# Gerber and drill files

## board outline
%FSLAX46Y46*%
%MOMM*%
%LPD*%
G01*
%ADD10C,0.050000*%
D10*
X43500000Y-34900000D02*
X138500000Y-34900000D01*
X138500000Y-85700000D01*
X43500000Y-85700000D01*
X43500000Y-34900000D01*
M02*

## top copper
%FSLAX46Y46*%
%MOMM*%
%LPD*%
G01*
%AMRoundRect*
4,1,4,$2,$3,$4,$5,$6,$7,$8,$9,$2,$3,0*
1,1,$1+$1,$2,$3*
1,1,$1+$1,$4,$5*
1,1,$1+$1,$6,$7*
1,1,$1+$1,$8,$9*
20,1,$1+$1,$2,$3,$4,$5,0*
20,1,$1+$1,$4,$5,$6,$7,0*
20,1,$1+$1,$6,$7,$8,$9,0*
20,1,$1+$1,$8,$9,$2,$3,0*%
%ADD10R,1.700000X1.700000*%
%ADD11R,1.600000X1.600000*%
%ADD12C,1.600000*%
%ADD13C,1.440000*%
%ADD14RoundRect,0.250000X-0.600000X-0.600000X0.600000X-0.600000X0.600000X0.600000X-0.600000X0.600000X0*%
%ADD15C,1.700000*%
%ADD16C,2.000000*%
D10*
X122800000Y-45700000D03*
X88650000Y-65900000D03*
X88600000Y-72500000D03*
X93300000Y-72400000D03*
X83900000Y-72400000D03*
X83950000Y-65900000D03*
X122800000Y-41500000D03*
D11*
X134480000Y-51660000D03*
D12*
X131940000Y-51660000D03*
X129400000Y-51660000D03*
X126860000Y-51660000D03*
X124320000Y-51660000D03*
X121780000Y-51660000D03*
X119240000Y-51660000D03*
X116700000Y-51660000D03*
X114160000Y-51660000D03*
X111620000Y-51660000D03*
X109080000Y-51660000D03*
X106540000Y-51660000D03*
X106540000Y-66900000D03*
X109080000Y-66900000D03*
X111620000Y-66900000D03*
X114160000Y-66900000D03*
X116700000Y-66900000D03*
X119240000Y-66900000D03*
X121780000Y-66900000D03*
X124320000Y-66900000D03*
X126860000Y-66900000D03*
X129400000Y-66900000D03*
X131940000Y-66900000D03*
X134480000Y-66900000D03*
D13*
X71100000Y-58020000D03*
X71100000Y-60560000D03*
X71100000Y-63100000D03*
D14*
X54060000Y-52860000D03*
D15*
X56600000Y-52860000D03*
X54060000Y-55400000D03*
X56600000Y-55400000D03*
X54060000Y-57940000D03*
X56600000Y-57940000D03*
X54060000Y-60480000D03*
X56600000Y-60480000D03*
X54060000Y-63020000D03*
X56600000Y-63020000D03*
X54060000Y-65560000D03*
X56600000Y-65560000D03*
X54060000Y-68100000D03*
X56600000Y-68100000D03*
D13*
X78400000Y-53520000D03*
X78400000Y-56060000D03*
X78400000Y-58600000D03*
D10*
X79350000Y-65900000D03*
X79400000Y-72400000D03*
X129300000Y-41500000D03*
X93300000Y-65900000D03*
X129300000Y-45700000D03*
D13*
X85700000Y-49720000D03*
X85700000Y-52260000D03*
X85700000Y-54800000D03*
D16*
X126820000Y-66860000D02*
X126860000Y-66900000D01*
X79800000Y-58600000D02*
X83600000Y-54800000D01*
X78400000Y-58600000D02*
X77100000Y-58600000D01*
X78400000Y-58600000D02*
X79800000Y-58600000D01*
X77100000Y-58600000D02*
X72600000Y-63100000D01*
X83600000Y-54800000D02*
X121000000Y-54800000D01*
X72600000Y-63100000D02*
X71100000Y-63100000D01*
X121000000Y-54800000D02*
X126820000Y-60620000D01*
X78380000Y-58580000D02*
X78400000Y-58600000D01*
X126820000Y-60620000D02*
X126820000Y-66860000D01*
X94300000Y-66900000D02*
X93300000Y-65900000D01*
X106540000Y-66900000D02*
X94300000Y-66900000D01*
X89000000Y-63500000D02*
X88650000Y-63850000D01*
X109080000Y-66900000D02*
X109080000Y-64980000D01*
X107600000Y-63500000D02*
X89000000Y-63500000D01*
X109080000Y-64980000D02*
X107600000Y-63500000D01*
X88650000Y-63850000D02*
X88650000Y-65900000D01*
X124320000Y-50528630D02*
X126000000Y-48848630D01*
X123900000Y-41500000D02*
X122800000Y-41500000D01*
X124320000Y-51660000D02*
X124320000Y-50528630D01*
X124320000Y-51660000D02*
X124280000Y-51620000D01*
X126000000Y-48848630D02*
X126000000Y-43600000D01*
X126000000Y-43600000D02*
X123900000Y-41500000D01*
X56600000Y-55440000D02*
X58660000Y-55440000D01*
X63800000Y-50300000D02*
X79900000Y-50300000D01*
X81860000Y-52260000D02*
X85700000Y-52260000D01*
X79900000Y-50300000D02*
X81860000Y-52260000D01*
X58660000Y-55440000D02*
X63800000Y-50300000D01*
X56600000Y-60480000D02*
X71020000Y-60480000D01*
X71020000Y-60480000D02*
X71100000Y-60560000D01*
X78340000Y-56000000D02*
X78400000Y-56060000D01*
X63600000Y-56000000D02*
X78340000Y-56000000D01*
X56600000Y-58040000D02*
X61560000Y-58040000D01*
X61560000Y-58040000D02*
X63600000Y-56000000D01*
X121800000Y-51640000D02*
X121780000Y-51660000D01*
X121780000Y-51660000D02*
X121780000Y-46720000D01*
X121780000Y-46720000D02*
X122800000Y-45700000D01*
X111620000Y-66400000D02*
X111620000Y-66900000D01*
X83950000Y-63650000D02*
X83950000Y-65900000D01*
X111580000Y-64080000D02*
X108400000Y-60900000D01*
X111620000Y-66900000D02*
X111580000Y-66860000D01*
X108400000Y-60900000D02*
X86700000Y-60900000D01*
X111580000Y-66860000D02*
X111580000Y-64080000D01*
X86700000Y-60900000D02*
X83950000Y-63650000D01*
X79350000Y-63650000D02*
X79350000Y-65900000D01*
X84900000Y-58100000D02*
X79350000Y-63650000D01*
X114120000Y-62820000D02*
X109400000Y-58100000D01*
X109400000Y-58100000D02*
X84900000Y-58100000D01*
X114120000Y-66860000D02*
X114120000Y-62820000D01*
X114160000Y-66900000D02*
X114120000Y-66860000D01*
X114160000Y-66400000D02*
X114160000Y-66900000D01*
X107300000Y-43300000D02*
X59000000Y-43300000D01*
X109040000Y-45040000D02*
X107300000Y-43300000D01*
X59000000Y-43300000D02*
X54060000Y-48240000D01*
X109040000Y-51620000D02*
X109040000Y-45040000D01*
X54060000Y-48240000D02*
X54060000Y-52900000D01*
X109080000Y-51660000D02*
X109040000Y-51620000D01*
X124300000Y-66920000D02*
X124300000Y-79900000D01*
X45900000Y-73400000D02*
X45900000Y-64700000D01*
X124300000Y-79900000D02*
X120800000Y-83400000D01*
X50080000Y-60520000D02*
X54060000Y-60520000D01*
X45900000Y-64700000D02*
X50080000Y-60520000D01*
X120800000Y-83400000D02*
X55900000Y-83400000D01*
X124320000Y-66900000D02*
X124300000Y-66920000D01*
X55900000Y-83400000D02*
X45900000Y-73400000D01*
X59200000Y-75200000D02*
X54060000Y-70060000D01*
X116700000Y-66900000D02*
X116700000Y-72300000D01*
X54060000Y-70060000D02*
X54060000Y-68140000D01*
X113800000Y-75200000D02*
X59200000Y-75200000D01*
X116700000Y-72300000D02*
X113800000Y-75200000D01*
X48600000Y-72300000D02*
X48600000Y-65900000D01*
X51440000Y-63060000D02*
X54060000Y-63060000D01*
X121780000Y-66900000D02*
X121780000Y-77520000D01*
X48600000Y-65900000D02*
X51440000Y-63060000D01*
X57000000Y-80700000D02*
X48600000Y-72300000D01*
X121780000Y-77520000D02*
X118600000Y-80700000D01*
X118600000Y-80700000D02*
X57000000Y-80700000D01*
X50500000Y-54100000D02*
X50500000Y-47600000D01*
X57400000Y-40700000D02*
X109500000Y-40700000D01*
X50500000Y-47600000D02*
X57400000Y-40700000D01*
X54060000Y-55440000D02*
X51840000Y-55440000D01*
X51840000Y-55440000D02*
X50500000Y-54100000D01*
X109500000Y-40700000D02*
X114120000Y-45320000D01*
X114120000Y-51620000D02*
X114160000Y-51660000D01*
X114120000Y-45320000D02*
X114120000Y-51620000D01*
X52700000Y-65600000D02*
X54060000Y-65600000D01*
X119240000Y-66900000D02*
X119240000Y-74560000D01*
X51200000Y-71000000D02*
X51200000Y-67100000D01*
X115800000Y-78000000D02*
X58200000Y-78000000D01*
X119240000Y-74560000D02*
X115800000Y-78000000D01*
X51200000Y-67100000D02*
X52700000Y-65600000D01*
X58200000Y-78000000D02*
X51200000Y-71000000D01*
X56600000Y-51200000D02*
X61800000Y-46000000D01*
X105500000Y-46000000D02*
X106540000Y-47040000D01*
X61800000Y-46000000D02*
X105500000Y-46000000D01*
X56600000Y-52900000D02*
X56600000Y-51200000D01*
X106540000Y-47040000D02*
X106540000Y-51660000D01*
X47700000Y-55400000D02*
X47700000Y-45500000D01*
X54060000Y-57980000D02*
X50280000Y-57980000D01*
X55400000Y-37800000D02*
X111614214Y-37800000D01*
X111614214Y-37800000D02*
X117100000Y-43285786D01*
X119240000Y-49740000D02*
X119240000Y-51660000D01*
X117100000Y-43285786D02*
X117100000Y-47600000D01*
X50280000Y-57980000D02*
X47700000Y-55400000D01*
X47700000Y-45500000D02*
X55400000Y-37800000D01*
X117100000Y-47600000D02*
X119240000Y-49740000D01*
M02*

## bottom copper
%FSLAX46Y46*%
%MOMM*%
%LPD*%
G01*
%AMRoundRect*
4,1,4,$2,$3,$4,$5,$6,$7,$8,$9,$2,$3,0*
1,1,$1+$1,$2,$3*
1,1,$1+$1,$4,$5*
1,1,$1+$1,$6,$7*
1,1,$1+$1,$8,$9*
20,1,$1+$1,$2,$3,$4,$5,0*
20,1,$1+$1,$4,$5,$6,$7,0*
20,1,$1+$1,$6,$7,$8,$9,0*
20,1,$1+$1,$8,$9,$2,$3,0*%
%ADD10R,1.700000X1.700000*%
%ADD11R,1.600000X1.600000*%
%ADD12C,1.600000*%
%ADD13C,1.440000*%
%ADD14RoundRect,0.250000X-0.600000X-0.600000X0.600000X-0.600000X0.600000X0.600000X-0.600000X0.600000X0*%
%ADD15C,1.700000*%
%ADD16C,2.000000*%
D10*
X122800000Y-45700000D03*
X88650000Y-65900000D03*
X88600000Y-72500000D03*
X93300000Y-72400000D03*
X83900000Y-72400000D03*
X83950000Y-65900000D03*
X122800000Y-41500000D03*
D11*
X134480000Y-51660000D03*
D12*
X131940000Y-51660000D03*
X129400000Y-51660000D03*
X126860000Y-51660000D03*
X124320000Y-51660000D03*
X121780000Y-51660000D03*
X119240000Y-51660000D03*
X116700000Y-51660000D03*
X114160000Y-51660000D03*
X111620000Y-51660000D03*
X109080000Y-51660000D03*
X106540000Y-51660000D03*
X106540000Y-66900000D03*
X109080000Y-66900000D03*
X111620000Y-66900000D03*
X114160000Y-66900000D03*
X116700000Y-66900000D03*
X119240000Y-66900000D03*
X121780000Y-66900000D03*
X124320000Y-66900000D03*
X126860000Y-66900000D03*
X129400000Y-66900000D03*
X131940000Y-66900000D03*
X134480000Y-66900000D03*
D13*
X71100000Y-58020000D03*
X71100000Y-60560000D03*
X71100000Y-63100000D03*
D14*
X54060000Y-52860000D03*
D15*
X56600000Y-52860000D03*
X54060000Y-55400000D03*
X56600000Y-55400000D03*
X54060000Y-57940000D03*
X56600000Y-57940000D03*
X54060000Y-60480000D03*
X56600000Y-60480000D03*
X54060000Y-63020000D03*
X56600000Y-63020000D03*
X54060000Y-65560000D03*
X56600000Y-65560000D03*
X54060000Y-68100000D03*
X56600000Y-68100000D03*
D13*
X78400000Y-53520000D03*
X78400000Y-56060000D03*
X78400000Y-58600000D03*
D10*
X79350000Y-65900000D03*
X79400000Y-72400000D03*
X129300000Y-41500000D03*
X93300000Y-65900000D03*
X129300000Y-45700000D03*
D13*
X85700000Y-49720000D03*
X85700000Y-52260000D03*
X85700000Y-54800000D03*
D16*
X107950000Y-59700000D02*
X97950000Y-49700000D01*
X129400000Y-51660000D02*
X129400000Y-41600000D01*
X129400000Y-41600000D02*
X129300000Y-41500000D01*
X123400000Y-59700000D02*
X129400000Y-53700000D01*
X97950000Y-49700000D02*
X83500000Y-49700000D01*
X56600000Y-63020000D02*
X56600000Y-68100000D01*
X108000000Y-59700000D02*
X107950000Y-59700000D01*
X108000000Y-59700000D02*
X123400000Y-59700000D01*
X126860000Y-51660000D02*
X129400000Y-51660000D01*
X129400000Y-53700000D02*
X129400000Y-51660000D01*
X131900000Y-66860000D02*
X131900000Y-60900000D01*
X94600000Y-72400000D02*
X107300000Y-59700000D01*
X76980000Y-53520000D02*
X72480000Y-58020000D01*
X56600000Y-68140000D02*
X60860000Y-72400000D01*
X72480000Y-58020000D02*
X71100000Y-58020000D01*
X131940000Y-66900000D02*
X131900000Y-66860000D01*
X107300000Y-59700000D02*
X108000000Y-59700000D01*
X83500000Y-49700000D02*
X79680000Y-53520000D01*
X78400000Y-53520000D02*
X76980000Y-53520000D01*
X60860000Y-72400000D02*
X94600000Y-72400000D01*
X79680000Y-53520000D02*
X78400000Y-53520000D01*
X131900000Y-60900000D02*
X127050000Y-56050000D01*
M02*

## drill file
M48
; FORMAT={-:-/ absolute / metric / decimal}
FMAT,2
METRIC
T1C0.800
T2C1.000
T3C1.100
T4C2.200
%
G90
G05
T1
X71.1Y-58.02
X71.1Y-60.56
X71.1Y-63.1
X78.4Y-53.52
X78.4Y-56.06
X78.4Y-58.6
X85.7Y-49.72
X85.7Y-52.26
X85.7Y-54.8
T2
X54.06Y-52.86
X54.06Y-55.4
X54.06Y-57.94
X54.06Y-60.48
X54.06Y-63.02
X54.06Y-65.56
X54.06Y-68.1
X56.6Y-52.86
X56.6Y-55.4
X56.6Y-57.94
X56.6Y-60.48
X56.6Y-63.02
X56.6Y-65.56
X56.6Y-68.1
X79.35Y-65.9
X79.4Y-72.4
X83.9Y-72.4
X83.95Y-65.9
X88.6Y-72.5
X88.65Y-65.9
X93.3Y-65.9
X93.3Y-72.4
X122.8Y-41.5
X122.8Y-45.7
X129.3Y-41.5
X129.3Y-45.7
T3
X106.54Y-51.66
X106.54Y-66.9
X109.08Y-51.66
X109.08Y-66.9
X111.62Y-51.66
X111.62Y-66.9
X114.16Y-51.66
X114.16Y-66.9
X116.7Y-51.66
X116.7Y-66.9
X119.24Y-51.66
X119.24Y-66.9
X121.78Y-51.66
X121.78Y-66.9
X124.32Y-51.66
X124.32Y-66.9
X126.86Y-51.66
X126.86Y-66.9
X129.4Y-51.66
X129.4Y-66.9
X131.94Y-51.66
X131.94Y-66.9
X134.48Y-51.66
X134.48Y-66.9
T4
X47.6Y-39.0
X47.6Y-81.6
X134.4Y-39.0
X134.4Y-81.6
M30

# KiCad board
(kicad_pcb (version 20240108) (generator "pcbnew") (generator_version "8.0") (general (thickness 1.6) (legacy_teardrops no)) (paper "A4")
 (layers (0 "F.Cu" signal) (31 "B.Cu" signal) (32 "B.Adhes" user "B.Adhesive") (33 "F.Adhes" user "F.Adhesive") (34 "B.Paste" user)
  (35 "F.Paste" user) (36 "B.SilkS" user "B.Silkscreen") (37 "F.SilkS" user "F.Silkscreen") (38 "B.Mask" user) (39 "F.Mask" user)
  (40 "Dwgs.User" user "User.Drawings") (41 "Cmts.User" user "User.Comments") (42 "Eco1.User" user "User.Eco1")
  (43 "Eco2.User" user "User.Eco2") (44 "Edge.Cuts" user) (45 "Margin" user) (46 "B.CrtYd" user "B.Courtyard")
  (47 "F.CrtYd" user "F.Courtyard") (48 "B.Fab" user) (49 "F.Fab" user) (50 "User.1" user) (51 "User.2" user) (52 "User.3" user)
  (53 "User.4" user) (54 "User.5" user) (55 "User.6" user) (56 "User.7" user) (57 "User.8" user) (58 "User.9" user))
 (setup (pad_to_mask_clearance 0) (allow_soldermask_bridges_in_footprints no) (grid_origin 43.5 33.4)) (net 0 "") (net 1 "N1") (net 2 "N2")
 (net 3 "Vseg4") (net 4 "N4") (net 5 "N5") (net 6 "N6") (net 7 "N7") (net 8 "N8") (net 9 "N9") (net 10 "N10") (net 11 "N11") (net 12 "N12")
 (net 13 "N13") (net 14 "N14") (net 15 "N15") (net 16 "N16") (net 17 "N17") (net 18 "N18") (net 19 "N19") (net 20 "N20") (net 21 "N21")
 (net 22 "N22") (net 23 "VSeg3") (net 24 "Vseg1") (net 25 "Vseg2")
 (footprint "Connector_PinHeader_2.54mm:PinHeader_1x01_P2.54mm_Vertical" (layer "F.Cu") (at 122.8 45.7 180)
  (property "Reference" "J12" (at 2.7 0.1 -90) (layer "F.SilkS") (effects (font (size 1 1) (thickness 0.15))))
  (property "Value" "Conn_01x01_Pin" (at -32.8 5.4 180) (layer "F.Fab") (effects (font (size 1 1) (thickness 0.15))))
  (pad "1" thru_hole rect (at 0 0 180) (size 1.7 1.7) (drill 1) (layers "*.Cu" "*.Mask") (remove_unused_layers no) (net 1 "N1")))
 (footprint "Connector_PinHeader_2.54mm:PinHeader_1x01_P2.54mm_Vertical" (layer "F.Cu") (at 88.65 65.9 180)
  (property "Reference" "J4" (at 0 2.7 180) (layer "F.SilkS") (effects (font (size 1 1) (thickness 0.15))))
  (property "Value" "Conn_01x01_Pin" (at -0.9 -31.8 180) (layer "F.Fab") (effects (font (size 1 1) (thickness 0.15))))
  (pad "1" thru_hole rect (at 0 0 180) (size 1.7 1.7) (drill 1) (layers "*.Cu" "*.Mask") (remove_unused_layers no) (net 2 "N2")))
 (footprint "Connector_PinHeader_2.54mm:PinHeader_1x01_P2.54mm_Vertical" (layer "F.Cu") (at 88.6 72.5 180)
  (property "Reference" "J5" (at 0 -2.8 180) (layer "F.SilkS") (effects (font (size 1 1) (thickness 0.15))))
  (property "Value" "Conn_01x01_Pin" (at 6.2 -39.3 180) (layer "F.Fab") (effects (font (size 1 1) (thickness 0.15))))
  (pad "1" thru_hole rect (at 0 0 180) (size 1.7 1.7) (drill 1) (layers "*.Cu" "*.Mask") (remove_unused_layers no) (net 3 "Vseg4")))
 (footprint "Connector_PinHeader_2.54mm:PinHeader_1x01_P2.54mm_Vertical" (layer "F.Cu") (at 93.3 72.4 180)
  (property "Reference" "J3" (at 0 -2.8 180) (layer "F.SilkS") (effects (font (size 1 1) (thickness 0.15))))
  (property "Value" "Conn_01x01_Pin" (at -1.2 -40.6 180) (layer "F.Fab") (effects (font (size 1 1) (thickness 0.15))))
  (pad "1" thru_hole rect (at 0 0 180) (size 1.7 1.7) (drill 1) (layers "*.Cu" "*.Mask") (remove_unused_layers no) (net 3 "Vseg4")))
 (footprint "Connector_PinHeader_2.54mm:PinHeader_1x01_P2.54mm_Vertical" (layer "F.Cu") (at 83.9 72.4 180)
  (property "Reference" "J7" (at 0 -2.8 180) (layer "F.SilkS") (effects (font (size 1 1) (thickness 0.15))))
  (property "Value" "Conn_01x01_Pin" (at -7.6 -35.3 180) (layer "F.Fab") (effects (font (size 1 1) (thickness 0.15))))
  (pad "1" thru_hole rect (at 0 0 180) (size 1.7 1.7) (drill 1) (layers "*.Cu" "*.Mask") (remove_unused_layers no) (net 3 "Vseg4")))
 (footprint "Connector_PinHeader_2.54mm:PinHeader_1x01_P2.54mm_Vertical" (layer "F.Cu") (at 83.95 65.9 180)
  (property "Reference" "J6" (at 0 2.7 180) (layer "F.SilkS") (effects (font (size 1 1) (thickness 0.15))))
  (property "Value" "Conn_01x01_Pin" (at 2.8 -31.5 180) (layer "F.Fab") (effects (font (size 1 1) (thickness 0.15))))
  (pad "1" thru_hole rect (at 0 0 180) (size 1.7 1.7) (drill 1) (layers "*.Cu" "*.Mask") (remove_unused_layers no) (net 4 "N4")))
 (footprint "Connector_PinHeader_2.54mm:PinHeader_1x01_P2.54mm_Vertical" (layer "F.Cu") (at 122.8 41.5 180)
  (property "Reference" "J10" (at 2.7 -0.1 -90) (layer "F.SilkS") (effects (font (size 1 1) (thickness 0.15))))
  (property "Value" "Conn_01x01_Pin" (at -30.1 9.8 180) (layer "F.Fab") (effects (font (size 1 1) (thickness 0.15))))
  (pad "1" thru_hole rect (at 0 0 180) (size 1.7 1.7) (drill 1) (layers "*.Cu" "*.Mask") (remove_unused_layers no) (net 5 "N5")))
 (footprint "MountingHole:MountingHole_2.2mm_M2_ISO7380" (layer "F.Cu") (at 47.6 81.6)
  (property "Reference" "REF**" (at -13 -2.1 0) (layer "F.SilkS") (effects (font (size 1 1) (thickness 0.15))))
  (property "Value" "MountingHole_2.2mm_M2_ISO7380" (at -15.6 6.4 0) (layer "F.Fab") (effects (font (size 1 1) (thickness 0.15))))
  (pad "" np_thru_hole circle (at 0 0) (size 2.2 2.2) (drill 2.2) (layers "*.Cu" "*.Mask")))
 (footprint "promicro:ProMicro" (layer "F.Cu") (at 120.51 59.28 180)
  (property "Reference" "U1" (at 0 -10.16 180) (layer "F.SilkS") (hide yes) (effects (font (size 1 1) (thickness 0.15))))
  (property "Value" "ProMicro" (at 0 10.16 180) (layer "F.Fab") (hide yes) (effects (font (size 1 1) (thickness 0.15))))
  (pad "1" thru_hole rect (at -13.97 7.62 180) (size 1.6 1.6) (drill 1.1) (layers "*.Cu" "*.Mask" "F.SilkS") (remove_unused_layers no)
   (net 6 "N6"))
  (pad "2" thru_hole circle (at -11.43 7.62 180) (size 1.6 1.6) (drill 1.1) (layers "*.Cu" "*.Mask" "F.SilkS") (remove_unused_layers no)
   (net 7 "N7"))
  (pad "3" thru_hole circle (at -8.89 7.62 180) (size 1.6 1.6) (drill 1.1) (layers "*.Cu" "*.Mask" "F.SilkS") (remove_unused_layers no)
   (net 3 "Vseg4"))
  (pad "4" thru_hole circle (at -6.35 7.62 180) (size 1.6 1.6) (drill 1.1) (layers "*.Cu" "*.Mask" "F.SilkS") (remove_unused_layers no)
   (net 3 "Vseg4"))
  (pad "5" thru_hole circle (at -3.81 7.62 180) (size 1.6 1.6) (drill 1.1) (layers "*.Cu" "*.Mask" "F.SilkS") (remove_unused_layers no)
   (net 5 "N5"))
  (pad "6" thru_hole circle (at -1.27 7.62 180) (size 1.6 1.6) (drill 1.1) (layers "*.Cu" "*.Mask" "F.SilkS") (remove_unused_layers no)
   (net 1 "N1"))
  (pad "7" thru_hole circle (at 1.27 7.62 180) (size 1.6 1.6) (drill 1.1) (layers "*.Cu" "*.Mask" "F.SilkS") (remove_unused_layers no)
   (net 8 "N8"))
  (pad "8" thru_hole circle (at 3.81 7.62 180) (size 1.6 1.6) (drill 1.1) (layers "*.Cu" "*.Mask" "F.SilkS") (remove_unused_layers no)
   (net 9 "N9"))
  (pad "9" thru_hole circle (at 6.35 7.62 180) (size 1.6 1.6) (drill 1.1) (layers "*.Cu" "*.Mask" "F.SilkS") (remove_unused_layers no)
   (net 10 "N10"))
  (pad "10" thru_hole circle (at 8.89 7.62 180) (size 1.6 1.6) (drill 1.1) (layers "*.Cu" "*.Mask" "F.SilkS") (remove_unused_layers no)
   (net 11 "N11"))
  (pad "11" thru_hole circle (at 11.43 7.62 180) (size 1.6 1.6) (drill 1.1) (layers "*.Cu" "*.Mask" "F.SilkS") (remove_unused_layers no)
   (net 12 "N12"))
  (pad "12" thru_hole circle (at 13.97 7.62 180) (size 1.6 1.6) (drill 1.1) (layers "*.Cu" "*.Mask" "F.SilkS") (remove_unused_layers no)
   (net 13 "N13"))
  (pad "13" thru_hole circle (at 13.97 -7.62 180) (size 1.6 1.6) (drill 1.1) (layers "*.Cu" "*.Mask" "F.SilkS") (remove_unused_layers no)
   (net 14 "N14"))
  (pad "14" thru_hole circle (at 11.43 -7.62 180) (size 1.6 1.6) (drill 1.1) (layers "*.Cu" "*.Mask" "F.SilkS") (remove_unused_layers no)
   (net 2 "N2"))
  (pad "15" thru_hole circle (at 8.89 -7.62 180) (size 1.6 1.6) (drill 1.1) (layers "*.Cu" "*.Mask" "F.SilkS") (remove_unused_layers no)
   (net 4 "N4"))
  (pad "16" thru_hole circle (at 6.35 -7.62 180) (size 1.6 1.6) (drill 1.1) (layers "*.Cu" "*.Mask" "F.SilkS") (remove_unused_layers no)
   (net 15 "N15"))
  (pad "17" thru_hole circle (at 3.81 -7.62 180) (size 1.6 1.6) (drill 1.1) (layers "*.Cu" "*.Mask" "F.SilkS") (remove_unused_layers no)
   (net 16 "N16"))
  (pad "18" thru_hole circle (at 1.27 -7.62 180) (size 1.6 1.6) (drill 1.1) (layers "*.Cu" "*.Mask" "F.SilkS") (remove_unused_layers no)
   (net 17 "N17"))
  (pad "19" thru_hole circle (at -1.27 -7.62 180) (size 1.6 1.6) (drill 1.1) (layers "*.Cu" "*.Mask" "F.SilkS") (remove_unused_layers no)
   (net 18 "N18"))
  (pad "20" thru_hole circle (at -3.81 -7.62 180) (size 1.6 1.6) (drill 1.1) (layers "*.Cu" "*.Mask" "F.SilkS") (remove_unused_layers no)
   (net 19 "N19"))
  (pad "21" thru_hole circle (at -6.35 -7.62 180) (size 1.6 1.6) (drill 1.1) (layers "*.Cu" "*.Mask" "F.SilkS") (remove_unused_layers no)
   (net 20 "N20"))
  (pad "22" thru_hole circle (at -8.89 -7.62 180) (size 1.6 1.6) (drill 1.1) (layers "*.Cu" "*.Mask" "F.SilkS") (remove_unused_layers no)
   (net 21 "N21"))
  (pad "23" thru_hole circle (at -11.43 -7.62 180) (size 1.6 1.6) (drill 1.1) (layers "*.Cu" "*.Mask" "F.SilkS") (remove_unused_layers no)
   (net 3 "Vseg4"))
  (pad "24" thru_hole circle (at -13.97 -7.62 180) (size 1.6 1.6) (drill 1.1) (layers "*.Cu" "*.Mask" "F.SilkS") (remove_unused_layers no)
   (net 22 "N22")))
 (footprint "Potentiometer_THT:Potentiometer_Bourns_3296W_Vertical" (layer "F.Cu") (at 71.1 58.02 90)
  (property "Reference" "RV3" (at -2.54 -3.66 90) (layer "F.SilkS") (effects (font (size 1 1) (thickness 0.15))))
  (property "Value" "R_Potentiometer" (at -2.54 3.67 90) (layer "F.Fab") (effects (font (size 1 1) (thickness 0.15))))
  (pad "1" thru_hole circle (at 0 0 90) (size 1.44 1.44) (drill 0.8) (layers "*.Cu" "*.Mask") (remove_unused_layers no) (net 3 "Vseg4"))
  (pad "2" thru_hole circle (at -2.54 0 90) (size 1.44 1.44) (drill 0.8) (layers "*.Cu" "*.Mask") (remove_unused_layers no) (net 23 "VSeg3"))
  (pad "3" thru_hole circle (at -5.08 0 90) (size 1.44 1.44) (drill 0.8) (layers "*.Cu" "*.Mask") (remove_unused_layers no) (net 20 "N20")))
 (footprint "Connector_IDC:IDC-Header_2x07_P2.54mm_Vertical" (layer "F.Cu") (at 54.06 52.86)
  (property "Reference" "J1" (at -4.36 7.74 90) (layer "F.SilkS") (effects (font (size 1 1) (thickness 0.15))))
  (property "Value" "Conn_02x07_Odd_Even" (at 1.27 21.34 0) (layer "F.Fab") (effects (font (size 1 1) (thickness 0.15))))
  (pad "1" thru_hole roundrect (at 0 0) (size 1.7 1.7) (drill 1) (layers "*.Cu" "*.Mask") (remove_unused_layers no)
   (roundrect_rratio 0.147059) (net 12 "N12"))
  (pad "2" thru_hole circle (at 2.54 0) (size 1.7 1.7) (drill 1) (layers "*.Cu" "*.Mask") (remove_unused_layers no) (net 13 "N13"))
  (pad "3" thru_hole circle (at 0 2.54) (size 1.7 1.7) (drill 1) (layers "*.Cu" "*.Mask") (remove_unused_layers no) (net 10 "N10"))
  (pad "4" thru_hole circle (at 2.54 2.54) (size 1.7 1.7) (drill 1) (layers "*.Cu" "*.Mask") (remove_unused_layers no) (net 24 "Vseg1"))
  (pad "5" thru_hole circle (at 0 5.08) (size 1.7 1.7) (drill 1) (layers "*.Cu" "*.Mask") (remove_unused_layers no) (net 8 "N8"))
  (pad "6" thru_hole circle (at 2.54 5.08) (size 1.7 1.7) (drill 1) (layers "*.Cu" "*.Mask") (remove_unused_layers no) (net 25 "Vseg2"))
  (pad "7" thru_hole circle (at 0 7.62) (size 1.7 1.7) (drill 1) (layers "*.Cu" "*.Mask") (remove_unused_layers no) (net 19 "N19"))
  (pad "8" thru_hole circle (at 2.54 7.62) (size 1.7 1.7) (drill 1) (layers "*.Cu" "*.Mask") (remove_unused_layers no) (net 23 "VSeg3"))
  (pad "9" thru_hole circle (at 0 10.16) (size 1.7 1.7) (drill 1) (layers "*.Cu" "*.Mask") (remove_unused_layers no) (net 18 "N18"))
  (pad "10" thru_hole circle (at 2.54 10.16) (size 1.7 1.7) (drill 1) (layers "*.Cu" "*.Mask") (remove_unused_layers no) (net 3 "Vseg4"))
  (pad "11" thru_hole circle (at 0 12.7) (size 1.7 1.7) (drill 1) (layers "*.Cu" "*.Mask") (remove_unused_layers no) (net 17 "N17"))
  (pad "12" thru_hole circle (at 2.54 12.7) (size 1.7 1.7) (drill 1) (layers "*.Cu" "*.Mask") (remove_unused_layers no) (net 3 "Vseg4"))
  (pad "13" thru_hole circle (at 0 15.24) (size 1.7 1.7) (drill 1) (layers "*.Cu" "*.Mask") (remove_unused_layers no) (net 16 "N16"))
  (pad "14" thru_hole circle (at 2.54 15.24) (size 1.7 1.7) (drill 1) (layers "*.Cu" "*.Mask") (remove_unused_layers no) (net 3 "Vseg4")))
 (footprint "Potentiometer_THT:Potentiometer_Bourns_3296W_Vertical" (layer "F.Cu") (at 78.4 53.52 90)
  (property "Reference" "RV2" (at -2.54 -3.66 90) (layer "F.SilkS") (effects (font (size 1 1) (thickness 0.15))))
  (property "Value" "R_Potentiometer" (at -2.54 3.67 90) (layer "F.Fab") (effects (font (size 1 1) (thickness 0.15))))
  (pad "1" thru_hole circle (at 0 0 90) (size 1.44 1.44) (drill 0.8) (layers "*.Cu" "*.Mask") (remove_unused_layers no) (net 3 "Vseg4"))
  (pad "2" thru_hole circle (at -2.54 0 90) (size 1.44 1.44) (drill 0.8) (layers "*.Cu" "*.Mask") (remove_unused_layers no) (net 25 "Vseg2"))
  (pad "3" thru_hole circle (at -5.08 0 90) (size 1.44 1.44) (drill 0.8) (layers "*.Cu" "*.Mask") (remove_unused_layers no) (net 20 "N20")))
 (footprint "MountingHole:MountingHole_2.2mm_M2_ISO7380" (layer "F.Cu") (at 47.6 39)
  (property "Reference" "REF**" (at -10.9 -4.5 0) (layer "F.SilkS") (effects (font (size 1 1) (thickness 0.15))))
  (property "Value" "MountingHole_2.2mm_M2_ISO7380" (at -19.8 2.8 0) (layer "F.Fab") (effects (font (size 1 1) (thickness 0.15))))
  (pad "" np_thru_hole circle (at 0 0) (size 2.2 2.2) (drill 2.2) (layers "*.Cu" "*.Mask")))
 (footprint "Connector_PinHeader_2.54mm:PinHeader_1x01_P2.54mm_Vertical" (layer "F.Cu") (at 79.35 65.9 180)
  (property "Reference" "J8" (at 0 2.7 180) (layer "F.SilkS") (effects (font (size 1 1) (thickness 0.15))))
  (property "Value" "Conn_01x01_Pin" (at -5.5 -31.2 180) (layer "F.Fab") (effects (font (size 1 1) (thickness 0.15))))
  (pad "1" thru_hole rect (at 0 0 180) (size 1.7 1.7) (drill 1) (layers "*.Cu" "*.Mask") (remove_unused_layers no) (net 15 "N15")))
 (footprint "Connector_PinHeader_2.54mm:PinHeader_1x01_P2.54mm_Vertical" (layer "F.Cu") (at 79.4 72.4 180)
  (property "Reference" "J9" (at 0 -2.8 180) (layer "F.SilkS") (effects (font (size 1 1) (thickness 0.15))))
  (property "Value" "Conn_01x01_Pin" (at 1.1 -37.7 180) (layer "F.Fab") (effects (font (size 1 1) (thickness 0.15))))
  (pad "1" thru_hole rect (at 0 0 180) (size 1.7 1.7) (drill 1) (layers "*.Cu" "*.Mask") (remove_unused_layers no) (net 3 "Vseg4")))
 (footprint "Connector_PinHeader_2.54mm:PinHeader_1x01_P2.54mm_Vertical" (layer "F.Cu") (at 129.3 41.5 180)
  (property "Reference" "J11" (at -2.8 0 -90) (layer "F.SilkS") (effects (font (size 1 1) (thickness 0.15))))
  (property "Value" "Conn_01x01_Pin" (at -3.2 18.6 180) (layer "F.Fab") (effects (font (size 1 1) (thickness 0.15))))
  (pad "1" thru_hole rect (at 0 0 180) (size 1.7 1.7) (drill 1) (layers "*.Cu" "*.Mask") (remove_unused_layers no) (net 3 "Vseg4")))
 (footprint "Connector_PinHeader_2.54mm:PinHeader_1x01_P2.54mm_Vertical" (layer "F.Cu") (at 93.3 65.9 180)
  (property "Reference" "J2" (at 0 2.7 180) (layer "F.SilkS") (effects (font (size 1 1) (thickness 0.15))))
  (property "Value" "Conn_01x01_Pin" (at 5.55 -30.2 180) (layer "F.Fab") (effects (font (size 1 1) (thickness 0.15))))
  (pad "1" thru_hole rect (at 0 0 180) (size 1.7 1.7) (drill 1) (layers "*.Cu" "*.Mask") (remove_unused_layers no) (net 14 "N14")))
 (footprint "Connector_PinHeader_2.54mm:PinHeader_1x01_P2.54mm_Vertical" (layer "F.Cu") (at 129.3 45.7 180)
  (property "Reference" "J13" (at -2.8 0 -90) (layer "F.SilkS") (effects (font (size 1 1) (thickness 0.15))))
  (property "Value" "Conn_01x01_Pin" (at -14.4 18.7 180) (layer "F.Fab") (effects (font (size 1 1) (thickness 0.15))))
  (pad "1" thru_hole rect (at 0 0 180) (size 1.7 1.7) (drill 1) (layers "*.Cu" "*.Mask") (remove_unused_layers no) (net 3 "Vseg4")))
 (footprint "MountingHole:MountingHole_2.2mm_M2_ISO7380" (layer "F.Cu") (at 134.4 81.6)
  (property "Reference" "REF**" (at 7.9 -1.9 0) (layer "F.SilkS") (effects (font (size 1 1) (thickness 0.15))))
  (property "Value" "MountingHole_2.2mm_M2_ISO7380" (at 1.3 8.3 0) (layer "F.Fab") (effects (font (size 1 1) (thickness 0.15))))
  (pad "" np_thru_hole circle (at 0 0) (size 2.2 2.2) (drill 2.2) (layers "*.Cu" "*.Mask")))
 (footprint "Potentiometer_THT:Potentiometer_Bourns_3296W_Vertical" (layer "F.Cu") (at 85.7 49.72 90)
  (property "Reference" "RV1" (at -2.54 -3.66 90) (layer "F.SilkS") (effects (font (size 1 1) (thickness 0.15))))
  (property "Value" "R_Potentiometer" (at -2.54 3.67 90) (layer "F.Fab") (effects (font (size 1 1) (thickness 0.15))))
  (pad "1" thru_hole circle (at 0 0 90) (size 1.44 1.44) (drill 0.8) (layers "*.Cu" "*.Mask") (remove_unused_layers no) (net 3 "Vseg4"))
  (pad "2" thru_hole circle (at -2.54 0 90) (size 1.44 1.44) (drill 0.8) (layers "*.Cu" "*.Mask") (remove_unused_layers no) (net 24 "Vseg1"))
  (pad "3" thru_hole circle (at -5.08 0 90) (size 1.44 1.44) (drill 0.8) (layers "*.Cu" "*.Mask") (remove_unused_layers no) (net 20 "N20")))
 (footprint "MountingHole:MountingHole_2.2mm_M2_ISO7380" (layer "F.Cu") (at 134.4 39)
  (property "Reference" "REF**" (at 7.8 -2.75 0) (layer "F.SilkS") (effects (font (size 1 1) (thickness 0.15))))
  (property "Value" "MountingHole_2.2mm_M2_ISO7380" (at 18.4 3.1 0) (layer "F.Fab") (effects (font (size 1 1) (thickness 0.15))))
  (pad "" np_thru_hole circle (at 0 0) (size 2.2 2.2) (drill 2.2) (layers "*.Cu" "*.Mask")))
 (gr_rect (start 43.5 34.9) (end 138.5 85.7) (stroke (width 0.05) (type default)) (fill none) (layer "Edge.Cuts"))
 (segment (start 126.82 66.86) (end 126.86 66.9) (width 2) (layer "F.Cu") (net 20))
 (segment (start 79.8 58.6) (end 83.6 54.8) (width 2) (layer "F.Cu") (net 20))
 (segment (start 78.4 58.6) (end 77.1 58.6) (width 2) (layer "F.Cu") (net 20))
 (segment (start 78.4 58.6) (end 79.8 58.6) (width 2) (layer "F.Cu") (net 20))
 (segment (start 77.1 58.6) (end 72.6 63.1) (width 2) (layer "F.Cu") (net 20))
 (segment (start 83.6 54.8) (end 121 54.8) (width 2) (layer "F.Cu") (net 20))
 (segment (start 72.6 63.1) (end 71.1 63.1) (width 2) (layer "F.Cu") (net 20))
 (segment (start 121 54.8) (end 126.82 60.62) (width 2) (layer "F.Cu") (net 20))
 (segment (start 78.38 58.58) (end 78.4 58.6) (width 2) (layer "F.Cu") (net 20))
 (segment (start 126.82 60.62) (end 126.82 66.86) (width 2) (layer "F.Cu") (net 20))
 (segment (start 94.3 66.9) (end 93.3 65.9) (width 2) (layer "F.Cu") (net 14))
 (segment (start 106.54 66.9) (end 94.3 66.9) (width 2) (layer "F.Cu") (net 14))
 (segment (start 89 63.5) (end 88.65 63.85) (width 2) (layer "F.Cu") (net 2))
 (segment (start 109.08 66.9) (end 109.08 64.98) (width 2) (layer "F.Cu") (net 2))
 (segment (start 107.6 63.5) (end 89 63.5) (width 2) (layer "F.Cu") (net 2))
 (segment (start 109.08 64.98) (end 107.6 63.5) (width 2) (layer "F.Cu") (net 2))
 (segment (start 88.65 63.85) (end 88.65 65.9) (width 2) (layer "F.Cu") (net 2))
 (segment (start 124.32 50.52863) (end 126 48.84863) (width 2) (layer "F.Cu") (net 5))
 (segment (start 123.9 41.5) (end 122.8 41.5) (width 2) (layer "F.Cu") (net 5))
 (segment (start 124.32 51.66) (end 124.32 50.52863) (width 2) (layer "F.Cu") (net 5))
 (segment (start 124.32 51.66) (end 124.28 51.62) (width 2) (layer "F.Cu") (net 5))
 (segment (start 126 48.84863) (end 126 43.6) (width 2) (layer "F.Cu") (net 5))
 (segment (start 126 43.6) (end 123.9 41.5) (width 2) (layer "F.Cu") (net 5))
 (segment (start 56.6 55.44) (end 58.66 55.44) (width 2) (layer "F.Cu") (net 24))
 (segment (start 63.8 50.3) (end 79.9 50.3) (width 2) (layer "F.Cu") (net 24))
 (segment (start 81.86 52.26) (end 85.7 52.26) (width 2) (layer "F.Cu") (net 24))
 (segment (start 79.9 50.3) (end 81.86 52.26) (width 2) (layer "F.Cu") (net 24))
 (segment (start 58.66 55.44) (end 63.8 50.3) (width 2) (layer "F.Cu") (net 24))
 (segment (start 56.6 60.48) (end 71.02 60.48) (width 2) (layer "F.Cu") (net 23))
 (segment (start 71.02 60.48) (end 71.1 60.56) (width 2) (layer "F.Cu") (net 23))
 (segment (start 107.95 59.7) (end 97.95 49.7) (width 2) (layer "B.Cu") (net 3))
 (segment (start 129.4 51.66) (end 129.4 41.6) (width 2) (layer "B.Cu") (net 3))
 (segment (start 129.4 41.6) (end 129.3 41.5) (width 2) (layer "B.Cu") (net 3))
 (segment (start 123.4 59.7) (end 129.4 53.7) (width 2) (layer "B.Cu") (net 3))
 (segment (start 97.95 49.7) (end 83.5 49.7) (width 2) (layer "B.Cu") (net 3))
 (segment (start 56.6 63.02) (end 56.6 68.1) (width 2) (layer "B.Cu") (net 3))
 (segment (start 108 59.7) (end 107.95 59.7) (width 2) (layer "B.Cu") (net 3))
 (segment (start 108 59.7) (end 123.4 59.7) (width 2) (layer "B.Cu") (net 3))
 (segment (start 126.86 51.66) (end 129.4 51.66) (width 2) (layer "B.Cu") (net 3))
 (segment (start 129.4 53.7) (end 129.4 51.66) (width 2) (layer "B.Cu") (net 3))
 (segment (start 131.9 66.86) (end 131.9 60.9) (width 2) (layer "B.Cu") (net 3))
 (segment (start 94.6 72.4) (end 107.3 59.7) (width 2) (layer "B.Cu") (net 3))
 (segment (start 76.98 53.52) (end 72.48 58.02) (width 2) (layer "B.Cu") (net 3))
 (segment (start 56.6 68.14) (end 60.86 72.4) (width 2) (layer "B.Cu") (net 3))
 (segment (start 72.48 58.02) (end 71.1 58.02) (width 2) (layer "B.Cu") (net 3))
 (segment (start 131.94 66.9) (end 131.9 66.86) (width 2) (layer "B.Cu") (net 3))
 (segment (start 107.3 59.7) (end 108 59.7) (width 2) (layer "B.Cu") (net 3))
 (segment (start 83.5 49.7) (end 79.68 53.52) (width 2) (layer "B.Cu") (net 3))
 (segment (start 78.4 53.52) (end 76.98 53.52) (width 2) (layer "B.Cu") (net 3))
 (segment (start 60.86 72.4) (end 94.6 72.4) (width 2) (layer "B.Cu") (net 3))
 (segment (start 79.68 53.52) (end 78.4 53.52) (width 2) (layer "B.Cu") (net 3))
 (segment (start 131.9 60.9) (end 127.05 56.05) (width 2) (layer "B.Cu") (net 3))
 (segment (start 78.34 56) (end 78.4 56.06) (width 2) (layer "F.Cu") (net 25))
 (segment (start 63.6 56) (end 78.34 56) (width 2) (layer "F.Cu") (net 25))
 (segment (start 56.6 58.04) (end 61.56 58.04) (width 2) (layer "F.Cu") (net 25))
 (segment (start 61.56 58.04) (end 63.6 56) (width 2) (layer "F.Cu") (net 25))
 (segment (start 121.8 51.64) (end 121.78 51.66) (width 2) (layer "F.Cu") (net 1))
 (segment (start 121.78 51.66) (end 121.78 46.72) (width 2) (layer "F.Cu") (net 1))
 (segment (start 121.78 46.72) (end 122.8 45.7) (width 2) (layer "F.Cu") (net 1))
 (segment (start 111.62 66.4) (end 111.62 66.9) (width 2) (layer "F.Cu") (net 4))
 (segment (start 83.95 63.65) (end 83.95 65.9) (width 2) (layer "F.Cu") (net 4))
 (segment (start 111.58 64.08) (end 108.4 60.9) (width 2) (layer "F.Cu") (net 4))
 (segment (start 111.62 66.9) (end 111.58 66.86) (width 2) (layer "F.Cu") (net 4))
 (segment (start 108.4 60.9) (end 86.7 60.9) (width 2) (layer "F.Cu") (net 4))
 (segment (start 111.58 66.86) (end 111.58 64.08) (width 2) (layer "F.Cu") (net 4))
 (segment (start 86.7 60.9) (end 83.95 63.65) (width 2) (layer "F.Cu") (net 4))
 (segment (start 79.35 63.65) (end 79.35 65.9) (width 2) (layer "F.Cu") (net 15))
 (segment (start 84.9 58.1) (end 79.35 63.65) (width 2) (layer "F.Cu") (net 15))
 (segment (start 114.12 62.82) (end 109.4 58.1) (width 2) (layer "F.Cu") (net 15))
 (segment (start 109.4 58.1) (end 84.9 58.1) (width 2) (layer "F.Cu") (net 15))
 (segment (start 114.12 66.86) (end 114.12 62.82) (width 2) (layer "F.Cu") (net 15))
 (segment (start 114.16 66.9) (end 114.12 66.86) (width 2) (layer "F.Cu") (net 15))
 (segment (start 114.16 66.4) (end 114.16 66.9) (width 2) (layer "F.Cu") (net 15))
 (segment (start 107.3 43.3) (end 59 43.3) (width 2) (layer "F.Cu") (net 12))
 (segment (start 109.04 45.04) (end 107.3 43.3) (width 2) (layer "F.Cu") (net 12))
 (segment (start 59 43.3) (end 54.06 48.24) (width 2) (layer "F.Cu") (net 12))
 (segment (start 109.04 51.62) (end 109.04 45.04) (width 2) (layer "F.Cu") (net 12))
 (segment (start 54.06 48.24) (end 54.06 52.9) (width 2) (layer "F.Cu") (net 12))
 (segment (start 109.08 51.66) (end 109.04 51.62) (width 2) (layer "F.Cu") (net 12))
 (segment (start 124.3 66.92) (end 124.3 79.9) (width 2) (layer "F.Cu") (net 19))
 (segment (start 45.9 73.4) (end 45.9 64.7) (width 2) (layer "F.Cu") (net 19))
 (segment (start 124.3 79.9) (end 120.8 83.4) (width 2) (layer "F.Cu") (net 19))
 (segment (start 50.08 60.52) (end 54.06 60.52) (width 2) (layer "F.Cu") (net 19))
 (segment (start 45.9 64.7) (end 50.08 60.52) (width 2) (layer "F.Cu") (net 19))
 (segment (start 120.8 83.4) (end 55.9 83.4) (width 2) (layer "F.Cu") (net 19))
 (segment (start 124.32 66.9) (end 124.3 66.92) (width 2) (layer "F.Cu") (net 19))
 (segment (start 55.9 83.4) (end 45.9 73.4) (width 2) (layer "F.Cu") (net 19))
 (segment (start 59.2 75.2) (end 54.06 70.06) (width 2) (layer "F.Cu") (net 16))
 (segment (start 116.7 66.9) (end 116.7 72.3) (width 2) (layer "F.Cu") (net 16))
 (segment (start 54.06 70.06) (end 54.06 68.14) (width 2) (layer "F.Cu") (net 16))
 (segment (start 113.8 75.2) (end 59.2 75.2) (width 2) (layer "F.Cu") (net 16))
 (segment (start 116.7 72.3) (end 113.8 75.2) (width 2) (layer "F.Cu") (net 16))
 (segment (start 48.6 72.3) (end 48.6 65.9) (width 2) (layer "F.Cu") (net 18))
 (segment (start 51.44 63.06) (end 54.06 63.06) (width 2) (layer "F.Cu") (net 18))
 (segment (start 121.78 66.9) (end 121.78 77.52) (width 2) (layer "F.Cu") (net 18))
 (segment (start 48.6 65.9) (end 51.44 63.06) (width 2) (layer "F.Cu") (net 18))
 (segment (start 57 80.7) (end 48.6 72.3) (width 2) (layer "F.Cu") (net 18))
 (segment (start 121.78 77.52) (end 118.6 80.7) (width 2) (layer "F.Cu") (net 18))
 (segment (start 118.6 80.7) (end 57 80.7) (width 2) (layer "F.Cu") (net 18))
 (segment (start 50.5 54.1) (end 50.5 47.6) (width 2) (layer "F.Cu") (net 10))
 (segment (start 57.4 40.7) (end 109.5 40.7) (width 2) (layer "F.Cu") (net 10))
 (segment (start 50.5 47.6) (end 57.4 40.7) (width 2) (layer "F.Cu") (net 10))
 (segment (start 54.06 55.44) (end 51.84 55.44) (width 2) (layer "F.Cu") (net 10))
 (segment (start 51.84 55.44) (end 50.5 54.1) (width 2) (layer "F.Cu") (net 10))
 (segment (start 109.5 40.7) (end 114.12 45.32) (width 2) (layer "F.Cu") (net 10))
 (segment (start 114.12 51.62) (end 114.16 51.66) (width 2) (layer "F.Cu") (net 10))
 (segment (start 114.12 45.32) (end 114.12 51.62) (width 2) (layer "F.Cu") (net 10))
 (segment (start 52.7 65.6) (end 54.06 65.6) (width 2) (layer "F.Cu") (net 17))
 (segment (start 119.24 66.9) (end 119.24 74.56) (width 2) (layer "F.Cu") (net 17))
 (segment (start 51.2 71) (end 51.2 67.1) (width 2) (layer "F.Cu") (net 17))
 (segment (start 115.8 78) (end 58.2 78) (width 2) (layer "F.Cu") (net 17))
 (segment (start 119.24 74.56) (end 115.8 78) (width 2) (layer "F.Cu") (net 17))
 (segment (start 51.2 67.1) (end 52.7 65.6) (width 2) (layer "F.Cu") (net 17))
 (segment (start 58.2 78) (end 51.2 71) (width 2) (layer "F.Cu") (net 17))
 (segment (start 56.6 51.2) (end 61.8 46) (width 2) (layer "F.Cu") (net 13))
 (segment (start 105.5 46) (end 106.54 47.04) (width 2) (layer "F.Cu") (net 13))
 (segment (start 61.8 46) (end 105.5 46) (width 2) (layer "F.Cu") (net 13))
 (segment (start 56.6 52.9) (end 56.6 51.2) (width 2) (layer "F.Cu") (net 13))
 (segment (start 106.54 47.04) (end 106.54 51.66) (width 2) (layer "F.Cu") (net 13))
 (segment (start 47.7 55.4) (end 47.7 45.5) (width 2) (layer "F.Cu") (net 8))
 (segment (start 54.06 57.98) (end 50.28 57.98) (width 2) (layer "F.Cu") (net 8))
 (segment (start 55.4 37.8) (end 111.614214 37.8) (width 2) (layer "F.Cu") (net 8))
 (segment (start 111.614214 37.8) (end 117.1 43.285786) (width 2) (layer "F.Cu") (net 8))
 (segment (start 119.24 49.74) (end 119.24 51.66) (width 2) (layer "F.Cu") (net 8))
 (segment (start 117.1 43.285786) (end 117.1 47.6) (width 2) (layer "F.Cu") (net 8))
 (segment (start 50.28 57.98) (end 47.7 55.4) (width 2) (layer "F.Cu") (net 8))
 (segment (start 47.7 45.5) (end 55.4 37.8) (width 2) (layer "F.Cu") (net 8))
 (segment (start 117.1 47.6) (end 119.24 49.74) (width 2) (layer "F.Cu") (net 8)))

